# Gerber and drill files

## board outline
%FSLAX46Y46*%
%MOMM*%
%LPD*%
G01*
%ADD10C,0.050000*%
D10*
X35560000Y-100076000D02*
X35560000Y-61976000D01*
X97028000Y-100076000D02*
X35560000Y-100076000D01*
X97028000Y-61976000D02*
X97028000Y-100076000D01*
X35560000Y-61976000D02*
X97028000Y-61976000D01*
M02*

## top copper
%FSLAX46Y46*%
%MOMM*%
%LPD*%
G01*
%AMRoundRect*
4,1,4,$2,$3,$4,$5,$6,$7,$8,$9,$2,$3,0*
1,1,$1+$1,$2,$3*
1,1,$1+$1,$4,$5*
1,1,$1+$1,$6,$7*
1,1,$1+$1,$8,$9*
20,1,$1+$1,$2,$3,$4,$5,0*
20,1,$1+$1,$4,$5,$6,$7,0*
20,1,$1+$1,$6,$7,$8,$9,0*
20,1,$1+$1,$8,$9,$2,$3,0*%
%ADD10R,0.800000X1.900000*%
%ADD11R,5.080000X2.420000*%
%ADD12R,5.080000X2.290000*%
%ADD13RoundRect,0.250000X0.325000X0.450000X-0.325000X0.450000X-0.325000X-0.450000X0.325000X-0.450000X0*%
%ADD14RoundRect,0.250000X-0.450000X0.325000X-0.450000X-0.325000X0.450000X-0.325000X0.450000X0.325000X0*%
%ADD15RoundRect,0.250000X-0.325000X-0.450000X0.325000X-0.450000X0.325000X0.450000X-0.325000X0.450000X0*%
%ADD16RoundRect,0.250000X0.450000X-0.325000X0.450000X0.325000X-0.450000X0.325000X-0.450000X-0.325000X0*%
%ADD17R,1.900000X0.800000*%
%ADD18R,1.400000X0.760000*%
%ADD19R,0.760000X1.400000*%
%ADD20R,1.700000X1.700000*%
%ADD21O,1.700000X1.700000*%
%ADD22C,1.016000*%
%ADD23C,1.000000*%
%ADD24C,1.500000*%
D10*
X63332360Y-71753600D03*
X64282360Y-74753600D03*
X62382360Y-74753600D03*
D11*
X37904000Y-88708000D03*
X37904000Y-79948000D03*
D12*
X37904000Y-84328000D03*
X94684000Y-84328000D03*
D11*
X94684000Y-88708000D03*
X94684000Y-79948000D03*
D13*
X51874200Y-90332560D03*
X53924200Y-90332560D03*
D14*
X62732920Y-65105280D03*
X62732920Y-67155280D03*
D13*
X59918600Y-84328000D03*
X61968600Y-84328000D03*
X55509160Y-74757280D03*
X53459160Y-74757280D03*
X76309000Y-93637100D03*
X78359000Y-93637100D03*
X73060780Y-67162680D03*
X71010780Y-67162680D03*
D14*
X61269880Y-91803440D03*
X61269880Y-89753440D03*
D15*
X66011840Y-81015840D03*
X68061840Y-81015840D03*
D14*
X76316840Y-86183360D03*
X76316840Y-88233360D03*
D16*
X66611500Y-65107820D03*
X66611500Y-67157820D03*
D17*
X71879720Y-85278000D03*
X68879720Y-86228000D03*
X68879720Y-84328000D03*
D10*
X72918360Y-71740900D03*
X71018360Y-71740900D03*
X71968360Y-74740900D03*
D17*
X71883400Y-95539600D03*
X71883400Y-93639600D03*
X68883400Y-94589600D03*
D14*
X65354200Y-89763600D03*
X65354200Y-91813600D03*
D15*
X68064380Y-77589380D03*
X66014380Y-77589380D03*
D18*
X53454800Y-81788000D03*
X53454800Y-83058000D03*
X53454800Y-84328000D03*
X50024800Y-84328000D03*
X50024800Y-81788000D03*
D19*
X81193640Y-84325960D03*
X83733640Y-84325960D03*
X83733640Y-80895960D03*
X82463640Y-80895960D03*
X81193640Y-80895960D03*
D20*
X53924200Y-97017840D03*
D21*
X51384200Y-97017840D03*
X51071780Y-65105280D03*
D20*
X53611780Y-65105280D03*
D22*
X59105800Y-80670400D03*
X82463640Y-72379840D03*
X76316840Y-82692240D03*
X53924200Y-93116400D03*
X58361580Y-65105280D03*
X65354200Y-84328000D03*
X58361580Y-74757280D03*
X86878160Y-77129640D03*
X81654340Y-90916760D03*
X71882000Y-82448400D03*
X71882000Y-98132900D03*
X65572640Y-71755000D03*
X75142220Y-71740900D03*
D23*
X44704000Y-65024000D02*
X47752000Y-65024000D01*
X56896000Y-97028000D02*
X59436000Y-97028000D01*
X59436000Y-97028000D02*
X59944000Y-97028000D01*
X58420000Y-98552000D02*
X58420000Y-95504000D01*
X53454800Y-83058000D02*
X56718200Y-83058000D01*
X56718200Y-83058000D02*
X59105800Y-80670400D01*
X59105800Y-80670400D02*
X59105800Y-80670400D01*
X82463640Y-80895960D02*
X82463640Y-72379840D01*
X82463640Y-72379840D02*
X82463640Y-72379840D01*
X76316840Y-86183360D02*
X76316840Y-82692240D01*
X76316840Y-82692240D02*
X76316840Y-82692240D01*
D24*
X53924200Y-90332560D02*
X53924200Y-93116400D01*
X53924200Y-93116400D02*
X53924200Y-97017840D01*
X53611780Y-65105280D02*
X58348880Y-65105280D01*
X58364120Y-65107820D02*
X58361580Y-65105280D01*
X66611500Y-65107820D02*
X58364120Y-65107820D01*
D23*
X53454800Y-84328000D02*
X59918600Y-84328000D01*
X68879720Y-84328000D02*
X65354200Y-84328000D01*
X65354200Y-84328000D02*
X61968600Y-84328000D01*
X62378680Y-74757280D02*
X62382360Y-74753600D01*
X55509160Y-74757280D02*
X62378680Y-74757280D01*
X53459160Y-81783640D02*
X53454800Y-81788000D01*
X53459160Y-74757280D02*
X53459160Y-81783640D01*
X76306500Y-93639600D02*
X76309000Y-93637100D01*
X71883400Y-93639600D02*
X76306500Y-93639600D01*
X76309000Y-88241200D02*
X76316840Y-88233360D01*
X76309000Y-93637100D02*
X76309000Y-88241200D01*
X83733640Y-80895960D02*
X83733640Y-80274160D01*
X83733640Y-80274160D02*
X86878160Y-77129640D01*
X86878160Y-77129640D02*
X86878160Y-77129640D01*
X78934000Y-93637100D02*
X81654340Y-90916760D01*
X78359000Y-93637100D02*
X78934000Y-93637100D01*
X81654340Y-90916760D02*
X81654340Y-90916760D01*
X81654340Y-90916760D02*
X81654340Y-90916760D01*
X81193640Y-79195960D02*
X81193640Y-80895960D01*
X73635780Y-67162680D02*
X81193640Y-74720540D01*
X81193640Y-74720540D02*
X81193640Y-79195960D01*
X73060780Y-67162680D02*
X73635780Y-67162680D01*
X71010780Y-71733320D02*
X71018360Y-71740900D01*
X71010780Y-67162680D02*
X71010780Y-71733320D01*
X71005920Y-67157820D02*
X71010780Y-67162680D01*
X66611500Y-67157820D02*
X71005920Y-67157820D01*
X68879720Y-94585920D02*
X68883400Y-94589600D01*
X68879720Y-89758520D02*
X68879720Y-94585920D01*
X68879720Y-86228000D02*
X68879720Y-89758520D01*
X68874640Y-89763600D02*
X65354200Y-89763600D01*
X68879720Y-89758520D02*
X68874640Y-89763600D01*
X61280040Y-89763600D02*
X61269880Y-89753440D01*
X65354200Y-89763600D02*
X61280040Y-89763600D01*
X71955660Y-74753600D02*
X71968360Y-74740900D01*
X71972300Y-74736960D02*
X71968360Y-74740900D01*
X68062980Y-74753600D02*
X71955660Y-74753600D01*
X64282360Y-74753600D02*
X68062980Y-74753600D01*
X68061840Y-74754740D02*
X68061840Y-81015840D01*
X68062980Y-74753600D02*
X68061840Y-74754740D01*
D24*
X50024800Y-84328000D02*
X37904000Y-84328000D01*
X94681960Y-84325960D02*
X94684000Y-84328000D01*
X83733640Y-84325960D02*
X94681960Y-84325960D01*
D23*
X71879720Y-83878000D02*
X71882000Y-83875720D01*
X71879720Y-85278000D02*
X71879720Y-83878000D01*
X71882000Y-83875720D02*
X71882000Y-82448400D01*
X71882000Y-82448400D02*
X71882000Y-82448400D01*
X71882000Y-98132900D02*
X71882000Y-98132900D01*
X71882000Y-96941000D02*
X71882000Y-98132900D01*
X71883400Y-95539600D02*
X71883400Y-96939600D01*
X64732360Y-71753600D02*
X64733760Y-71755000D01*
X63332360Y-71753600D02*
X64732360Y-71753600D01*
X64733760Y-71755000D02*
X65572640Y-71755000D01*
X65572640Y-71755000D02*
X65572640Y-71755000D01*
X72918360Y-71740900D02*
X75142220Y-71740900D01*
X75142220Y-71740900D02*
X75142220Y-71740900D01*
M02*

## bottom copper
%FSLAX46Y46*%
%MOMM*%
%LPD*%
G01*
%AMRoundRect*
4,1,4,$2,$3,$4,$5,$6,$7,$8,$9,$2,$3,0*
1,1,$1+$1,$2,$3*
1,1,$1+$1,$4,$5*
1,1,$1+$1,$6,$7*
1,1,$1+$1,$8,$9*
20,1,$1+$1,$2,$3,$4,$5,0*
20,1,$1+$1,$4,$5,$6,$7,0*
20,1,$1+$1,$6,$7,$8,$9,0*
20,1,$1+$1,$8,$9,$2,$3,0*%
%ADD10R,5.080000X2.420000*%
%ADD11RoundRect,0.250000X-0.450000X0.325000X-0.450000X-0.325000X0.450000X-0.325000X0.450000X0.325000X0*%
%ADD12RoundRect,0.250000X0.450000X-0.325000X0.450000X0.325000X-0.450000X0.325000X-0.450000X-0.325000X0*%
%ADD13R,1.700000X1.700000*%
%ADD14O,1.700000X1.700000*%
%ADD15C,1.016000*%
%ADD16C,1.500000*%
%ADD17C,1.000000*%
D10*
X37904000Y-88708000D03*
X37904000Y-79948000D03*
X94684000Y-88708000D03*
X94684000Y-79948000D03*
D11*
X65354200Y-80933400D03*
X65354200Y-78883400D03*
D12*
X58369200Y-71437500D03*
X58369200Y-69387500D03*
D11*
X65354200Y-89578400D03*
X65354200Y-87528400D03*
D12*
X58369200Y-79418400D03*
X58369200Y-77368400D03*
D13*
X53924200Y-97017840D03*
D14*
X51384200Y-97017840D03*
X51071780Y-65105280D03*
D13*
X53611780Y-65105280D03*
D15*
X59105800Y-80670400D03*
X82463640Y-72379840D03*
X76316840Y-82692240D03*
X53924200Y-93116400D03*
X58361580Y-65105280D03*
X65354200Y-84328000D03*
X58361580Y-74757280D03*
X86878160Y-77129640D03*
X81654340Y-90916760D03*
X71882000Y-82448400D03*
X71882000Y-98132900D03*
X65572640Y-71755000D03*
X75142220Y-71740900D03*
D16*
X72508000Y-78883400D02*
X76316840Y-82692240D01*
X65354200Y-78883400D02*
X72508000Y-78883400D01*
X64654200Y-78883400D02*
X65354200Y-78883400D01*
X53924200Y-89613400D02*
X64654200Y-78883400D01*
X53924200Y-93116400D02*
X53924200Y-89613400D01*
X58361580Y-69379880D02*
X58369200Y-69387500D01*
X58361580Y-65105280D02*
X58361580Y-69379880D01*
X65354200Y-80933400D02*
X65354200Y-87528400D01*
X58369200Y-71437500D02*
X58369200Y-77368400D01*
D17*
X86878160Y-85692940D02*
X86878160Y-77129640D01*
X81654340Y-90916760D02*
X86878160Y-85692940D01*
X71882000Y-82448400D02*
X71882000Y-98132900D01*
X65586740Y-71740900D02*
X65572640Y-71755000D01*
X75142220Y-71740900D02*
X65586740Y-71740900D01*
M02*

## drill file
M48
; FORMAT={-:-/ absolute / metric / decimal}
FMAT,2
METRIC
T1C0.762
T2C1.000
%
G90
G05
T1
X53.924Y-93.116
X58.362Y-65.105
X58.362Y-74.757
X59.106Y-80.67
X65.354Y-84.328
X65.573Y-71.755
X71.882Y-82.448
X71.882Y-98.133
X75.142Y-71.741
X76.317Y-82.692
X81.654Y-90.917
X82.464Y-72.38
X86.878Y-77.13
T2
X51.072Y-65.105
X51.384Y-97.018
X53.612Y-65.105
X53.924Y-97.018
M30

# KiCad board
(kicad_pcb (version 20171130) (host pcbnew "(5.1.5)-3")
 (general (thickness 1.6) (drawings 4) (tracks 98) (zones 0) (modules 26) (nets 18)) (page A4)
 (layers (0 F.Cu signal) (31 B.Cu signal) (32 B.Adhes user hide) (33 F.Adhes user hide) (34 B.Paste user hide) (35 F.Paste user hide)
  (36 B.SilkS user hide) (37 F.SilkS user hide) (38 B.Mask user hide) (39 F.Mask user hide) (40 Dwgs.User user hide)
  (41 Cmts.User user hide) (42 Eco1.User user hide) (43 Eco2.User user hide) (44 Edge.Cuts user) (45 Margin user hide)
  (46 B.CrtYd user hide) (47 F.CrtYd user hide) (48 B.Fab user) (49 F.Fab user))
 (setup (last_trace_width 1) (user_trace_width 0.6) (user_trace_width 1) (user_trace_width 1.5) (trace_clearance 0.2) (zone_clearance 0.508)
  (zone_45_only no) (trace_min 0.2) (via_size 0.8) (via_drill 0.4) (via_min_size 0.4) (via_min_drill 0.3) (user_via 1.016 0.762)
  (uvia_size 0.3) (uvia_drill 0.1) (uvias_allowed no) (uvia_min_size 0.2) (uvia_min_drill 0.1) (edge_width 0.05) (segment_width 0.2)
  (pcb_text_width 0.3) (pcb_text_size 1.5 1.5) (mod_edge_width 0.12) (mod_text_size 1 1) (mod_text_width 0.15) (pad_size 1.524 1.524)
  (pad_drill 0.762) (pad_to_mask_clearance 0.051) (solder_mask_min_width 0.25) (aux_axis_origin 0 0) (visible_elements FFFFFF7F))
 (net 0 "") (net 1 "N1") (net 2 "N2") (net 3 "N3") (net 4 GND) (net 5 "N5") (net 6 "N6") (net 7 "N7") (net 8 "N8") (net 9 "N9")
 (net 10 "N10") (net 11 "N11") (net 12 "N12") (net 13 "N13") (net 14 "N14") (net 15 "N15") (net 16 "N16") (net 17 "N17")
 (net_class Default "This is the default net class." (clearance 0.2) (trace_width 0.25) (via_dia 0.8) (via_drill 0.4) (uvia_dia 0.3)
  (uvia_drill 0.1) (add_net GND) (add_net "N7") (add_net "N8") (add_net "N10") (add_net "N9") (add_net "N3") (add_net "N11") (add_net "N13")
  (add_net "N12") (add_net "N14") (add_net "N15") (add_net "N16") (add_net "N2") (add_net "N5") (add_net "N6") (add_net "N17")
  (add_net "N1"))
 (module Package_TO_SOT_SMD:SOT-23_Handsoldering (layer F.Cu) (at 63.33236 73.2536 90)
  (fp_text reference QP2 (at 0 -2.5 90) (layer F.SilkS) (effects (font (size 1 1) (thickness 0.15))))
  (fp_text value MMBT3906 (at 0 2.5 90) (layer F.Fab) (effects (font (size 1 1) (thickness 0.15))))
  (pad 3 smd rect (at 1.5 0 90) (size 1.9 0.8) (layers F.Cu F.Paste F.Mask) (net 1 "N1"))
  (pad 2 smd rect (at -1.5 0.95 90) (size 1.9 0.8) (layers F.Cu F.Paste F.Mask) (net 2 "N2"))
  (pad 1 smd rect (at -1.5 -0.95 90) (size 1.9 0.8) (layers F.Cu F.Paste F.Mask) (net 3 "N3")))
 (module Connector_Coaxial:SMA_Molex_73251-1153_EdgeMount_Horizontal (layer F.Cu) (at 39.624 84.328)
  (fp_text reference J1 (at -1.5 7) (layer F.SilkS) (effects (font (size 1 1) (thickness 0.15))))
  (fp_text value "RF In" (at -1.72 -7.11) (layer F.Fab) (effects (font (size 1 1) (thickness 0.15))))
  (pad 2 smd rect (at -1.72 4.38) (size 5.08 2.42) (layers B.Cu B.Paste B.Mask) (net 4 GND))
  (pad 2 smd rect (at -1.72 -4.38) (size 5.08 2.42) (layers B.Cu B.Paste B.Mask) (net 4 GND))
  (pad 2 smd rect (at -1.72 4.38) (size 5.08 2.42) (layers F.Cu F.Paste F.Mask) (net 4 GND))
  (pad 2 smd rect (at -1.72 -4.38) (size 5.08 2.42) (layers F.Cu F.Paste F.Mask) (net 4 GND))
  (pad 1 smd rect (at -1.72 0) (size 5.08 2.29) (layers F.Cu F.Paste F.Mask) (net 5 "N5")))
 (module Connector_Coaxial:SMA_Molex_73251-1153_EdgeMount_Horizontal (layer F.Cu) (at 92.964 84.328 180)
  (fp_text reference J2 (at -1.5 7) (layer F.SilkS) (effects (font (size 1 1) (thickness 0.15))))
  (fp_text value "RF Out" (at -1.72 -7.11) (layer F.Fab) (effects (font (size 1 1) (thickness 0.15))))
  (pad 1 smd rect (at -1.72 0 180) (size 5.08 2.29) (layers F.Cu F.Paste F.Mask) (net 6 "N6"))
  (pad 2 smd rect (at -1.72 -4.38 180) (size 5.08 2.42) (layers F.Cu F.Paste F.Mask) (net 4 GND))
  (pad 2 smd rect (at -1.72 4.38 180) (size 5.08 2.42) (layers F.Cu F.Paste F.Mask) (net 4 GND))
  (pad 2 smd rect (at -1.72 -4.38 180) (size 5.08 2.42) (layers B.Cu B.Paste B.Mask) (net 4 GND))
  (pad 2 smd rect (at -1.72 4.38 180) (size 5.08 2.42) (layers B.Cu B.Paste B.Mask) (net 4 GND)))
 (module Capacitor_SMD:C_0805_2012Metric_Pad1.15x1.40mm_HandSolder (layer F.Cu) (at 52.8992 90.33256 180)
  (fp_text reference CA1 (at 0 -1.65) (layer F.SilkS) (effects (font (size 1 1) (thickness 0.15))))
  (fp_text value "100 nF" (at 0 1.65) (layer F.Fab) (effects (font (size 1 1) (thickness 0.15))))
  (pad 2 smd roundrect (at 1.025 0 180) (size 1.15 1.4) (layers F.Cu F.Paste F.Mask) (roundrect_rratio 0.217391) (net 4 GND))
  (pad 1 smd roundrect (at -1.025 0 180) (size 1.15 1.4) (layers F.Cu F.Paste F.Mask) (roundrect_rratio 0.217391) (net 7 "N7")))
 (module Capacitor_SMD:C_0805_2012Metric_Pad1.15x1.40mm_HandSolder (layer F.Cu) (at 62.73292 66.13028 270)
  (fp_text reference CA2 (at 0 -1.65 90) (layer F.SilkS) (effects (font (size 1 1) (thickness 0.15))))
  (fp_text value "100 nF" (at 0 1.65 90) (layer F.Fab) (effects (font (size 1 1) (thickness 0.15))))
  (pad 1 smd roundrect (at -1.025 0 270) (size 1.15 1.4) (layers F.Cu F.Paste F.Mask) (roundrect_rratio 0.217391) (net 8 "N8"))
  (pad 2 smd roundrect (at 1.025 0 270) (size 1.15 1.4) (layers F.Cu F.Paste F.Mask) (roundrect_rratio 0.217391) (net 4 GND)))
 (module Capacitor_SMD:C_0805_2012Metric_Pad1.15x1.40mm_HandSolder (layer F.Cu) (at 60.9436 84.328 180)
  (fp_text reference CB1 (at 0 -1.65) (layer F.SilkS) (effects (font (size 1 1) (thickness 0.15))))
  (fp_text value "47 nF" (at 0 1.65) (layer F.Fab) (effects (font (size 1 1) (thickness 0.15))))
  (pad 2 smd roundrect (at 1.025 0 180) (size 1.15 1.4) (layers F.Cu F.Paste F.Mask) (roundrect_rratio 0.217391) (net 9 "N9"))
  (pad 1 smd roundrect (at -1.025 0 180) (size 1.15 1.4) (layers F.Cu F.Paste F.Mask) (roundrect_rratio 0.217391) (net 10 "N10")))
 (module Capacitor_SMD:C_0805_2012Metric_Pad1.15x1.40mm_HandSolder (layer F.Cu) (at 54.48416 74.75728 180)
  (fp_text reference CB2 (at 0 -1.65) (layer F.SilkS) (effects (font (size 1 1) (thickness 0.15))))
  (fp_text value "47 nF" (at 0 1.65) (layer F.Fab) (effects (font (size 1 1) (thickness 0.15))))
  (pad 1 smd roundrect (at -1.025 0 180) (size 1.15 1.4) (layers F.Cu F.Paste F.Mask) (roundrect_rratio 0.217391) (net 3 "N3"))
  (pad 2 smd roundrect (at 1.025 0 180) (size 1.15 1.4) (layers F.Cu F.Paste F.Mask) (roundrect_rratio 0.217391) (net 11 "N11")))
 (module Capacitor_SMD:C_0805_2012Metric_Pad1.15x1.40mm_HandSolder (layer F.Cu) (at 77.334 93.6371 180)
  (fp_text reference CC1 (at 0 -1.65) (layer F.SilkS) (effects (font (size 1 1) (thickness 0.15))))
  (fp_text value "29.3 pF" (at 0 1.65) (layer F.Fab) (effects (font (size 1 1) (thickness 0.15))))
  (pad 2 smd roundrect (at 1.025 0 180) (size 1.15 1.4) (layers F.Cu F.Paste F.Mask) (roundrect_rratio 0.217391) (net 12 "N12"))
  (pad 1 smd roundrect (at -1.025 0 180) (size 1.15 1.4) (layers F.Cu F.Paste F.Mask) (roundrect_rratio 0.217391) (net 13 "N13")))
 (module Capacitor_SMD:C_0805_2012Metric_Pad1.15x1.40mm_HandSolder (layer F.Cu) (at 72.03578 67.16268 180)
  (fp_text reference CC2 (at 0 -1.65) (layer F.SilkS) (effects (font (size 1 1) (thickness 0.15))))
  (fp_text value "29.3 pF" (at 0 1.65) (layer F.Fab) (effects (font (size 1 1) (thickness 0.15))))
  (pad 1 smd roundrect (at -1.025 0 180) (size 1.15 1.4) (layers F.Cu F.Paste F.Mask) (roundrect_rratio 0.217391) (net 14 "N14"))
  (pad 2 smd roundrect (at 1.025 0 180) (size 1.15 1.4) (layers F.Cu F.Paste F.Mask) (roundrect_rratio 0.217391) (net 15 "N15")))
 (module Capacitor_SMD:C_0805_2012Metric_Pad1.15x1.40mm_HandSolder (layer F.Cu) (at 61.26988 90.77844 270)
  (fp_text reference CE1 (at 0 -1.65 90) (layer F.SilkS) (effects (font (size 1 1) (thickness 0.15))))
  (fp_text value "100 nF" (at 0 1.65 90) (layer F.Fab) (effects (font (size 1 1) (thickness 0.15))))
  (pad 2 smd roundrect (at 1.025 0 270) (size 1.15 1.4) (layers F.Cu F.Paste F.Mask) (roundrect_rratio 0.217391) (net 4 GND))
  (pad 1 smd roundrect (at -1.025 0 270) (size 1.15 1.4) (layers F.Cu F.Paste F.Mask) (roundrect_rratio 0.217391) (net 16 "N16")))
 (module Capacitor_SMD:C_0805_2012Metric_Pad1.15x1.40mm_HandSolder (layer F.Cu) (at 67.03684 81.01584)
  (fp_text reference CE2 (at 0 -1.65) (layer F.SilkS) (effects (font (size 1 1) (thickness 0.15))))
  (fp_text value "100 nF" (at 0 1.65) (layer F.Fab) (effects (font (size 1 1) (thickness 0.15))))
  (pad 1 smd roundrect (at -1.025 0) (size 1.15 1.4) (layers F.Cu F.Paste F.Mask) (roundrect_rratio 0.217391) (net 4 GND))
  (pad 2 smd roundrect (at 1.025 0) (size 1.15 1.4) (layers F.Cu F.Paste F.Mask) (roundrect_rratio 0.217391) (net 2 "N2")))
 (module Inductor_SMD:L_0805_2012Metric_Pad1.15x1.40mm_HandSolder (layer F.Cu) (at 76.31684 87.20836 270)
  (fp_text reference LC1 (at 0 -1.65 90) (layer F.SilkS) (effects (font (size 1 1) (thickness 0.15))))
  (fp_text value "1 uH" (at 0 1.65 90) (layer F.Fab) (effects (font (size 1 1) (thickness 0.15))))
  (pad 1 smd roundrect (at -1.025 0 270) (size 1.15 1.4) (layers F.Cu F.Paste F.Mask) (roundrect_rratio 0.217391) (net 7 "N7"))
  (pad 2 smd roundrect (at 1.025 0 270) (size 1.15 1.4) (layers F.Cu F.Paste F.Mask) (roundrect_rratio 0.217391) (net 12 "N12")))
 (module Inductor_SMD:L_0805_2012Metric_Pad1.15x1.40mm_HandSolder (layer F.Cu) (at 66.6115 66.13282 90)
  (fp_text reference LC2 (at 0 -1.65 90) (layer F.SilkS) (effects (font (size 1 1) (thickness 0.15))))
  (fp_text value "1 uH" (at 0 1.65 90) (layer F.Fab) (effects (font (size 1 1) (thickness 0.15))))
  (pad 2 smd roundrect (at 1.025 0 90) (size 1.15 1.4) (layers F.Cu F.Paste F.Mask) (roundrect_rratio 0.217391) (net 8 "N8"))
  (pad 1 smd roundrect (at -1.025 0 90) (size 1.15 1.4) (layers F.Cu F.Paste F.Mask) (roundrect_rratio 0.217391) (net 15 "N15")))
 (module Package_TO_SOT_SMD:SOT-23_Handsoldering (layer F.Cu) (at 70.37972 85.278)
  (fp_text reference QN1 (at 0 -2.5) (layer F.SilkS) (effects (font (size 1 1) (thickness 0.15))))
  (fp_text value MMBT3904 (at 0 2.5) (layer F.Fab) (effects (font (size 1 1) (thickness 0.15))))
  (pad 3 smd rect (at 1.5 0) (size 1.9 0.8) (layers F.Cu F.Paste F.Mask) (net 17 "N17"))
  (pad 2 smd rect (at -1.5 0.95) (size 1.9 0.8) (layers F.Cu F.Paste F.Mask) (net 16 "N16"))
  (pad 1 smd rect (at -1.5 -0.95) (size 1.9 0.8) (layers F.Cu F.Paste F.Mask) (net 10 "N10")))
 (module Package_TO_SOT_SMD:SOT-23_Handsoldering (layer F.Cu) (at 71.96836 73.2409 270)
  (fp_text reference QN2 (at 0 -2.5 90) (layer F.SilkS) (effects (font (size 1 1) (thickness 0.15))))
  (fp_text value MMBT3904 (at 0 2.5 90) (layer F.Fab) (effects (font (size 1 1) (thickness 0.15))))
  (pad 1 smd rect (at -1.5 -0.95 270) (size 1.9 0.8) (layers F.Cu F.Paste F.Mask) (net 1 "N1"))
  (pad 2 smd rect (at -1.5 0.95 270) (size 1.9 0.8) (layers F.Cu F.Paste F.Mask) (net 15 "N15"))
  (pad 3 smd rect (at 1.5 0 270) (size 1.9 0.8) (layers F.Cu F.Paste F.Mask) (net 2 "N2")))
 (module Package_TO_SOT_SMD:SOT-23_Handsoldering (layer F.Cu) (at 70.3834 94.5896 180)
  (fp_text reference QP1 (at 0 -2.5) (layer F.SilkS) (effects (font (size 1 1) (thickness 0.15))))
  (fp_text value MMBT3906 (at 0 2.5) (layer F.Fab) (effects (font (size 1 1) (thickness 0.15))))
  (pad 1 smd rect (at -1.5 -0.95 180) (size 1.9 0.8) (layers F.Cu F.Paste F.Mask) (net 17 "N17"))
  (pad 2 smd rect (at -1.5 0.95 180) (size 1.9 0.8) (layers F.Cu F.Paste F.Mask) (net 12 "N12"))
  (pad 3 smd rect (at 1.5 0 180) (size 1.9 0.8) (layers F.Cu F.Paste F.Mask) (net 16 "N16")))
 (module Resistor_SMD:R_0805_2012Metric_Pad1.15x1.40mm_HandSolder (layer B.Cu) (at 65.3542 79.9084 270)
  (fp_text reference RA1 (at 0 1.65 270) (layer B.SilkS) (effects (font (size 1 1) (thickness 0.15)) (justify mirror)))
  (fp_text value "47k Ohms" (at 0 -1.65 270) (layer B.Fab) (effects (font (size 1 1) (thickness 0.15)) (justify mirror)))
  (pad 2 smd roundrect (at 1.025 0 270) (size 1.15 1.4) (layers B.Cu B.Paste B.Mask) (roundrect_rratio 0.217391) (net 10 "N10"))
  (pad 1 smd roundrect (at -1.025 0 270) (size 1.15 1.4) (layers B.Cu B.Paste B.Mask) (roundrect_rratio 0.217391) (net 7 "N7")))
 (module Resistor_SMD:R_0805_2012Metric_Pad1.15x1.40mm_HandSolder (layer B.Cu) (at 58.3692 70.4125 90)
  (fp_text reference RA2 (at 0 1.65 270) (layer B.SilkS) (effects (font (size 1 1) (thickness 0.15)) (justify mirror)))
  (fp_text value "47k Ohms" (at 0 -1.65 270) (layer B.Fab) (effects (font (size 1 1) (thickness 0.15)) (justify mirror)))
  (pad 1 smd roundrect (at -1.025 0 90) (size 1.15 1.4) (layers B.Cu B.Paste B.Mask) (roundrect_rratio 0.217391) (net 3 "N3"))
  (pad 2 smd roundrect (at 1.025 0 90) (size 1.15 1.4) (layers B.Cu B.Paste B.Mask) (roundrect_rratio 0.217391) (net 8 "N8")))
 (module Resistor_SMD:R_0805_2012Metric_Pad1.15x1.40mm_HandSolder (layer B.Cu) (at 65.3542 88.5534 270)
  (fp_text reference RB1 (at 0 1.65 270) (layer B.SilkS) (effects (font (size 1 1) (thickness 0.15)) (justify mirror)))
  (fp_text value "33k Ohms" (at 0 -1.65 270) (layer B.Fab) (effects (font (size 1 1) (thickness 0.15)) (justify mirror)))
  (pad 2 smd roundrect (at 1.025 0 270) (size 1.15 1.4) (layers B.Cu B.Paste B.Mask) (roundrect_rratio 0.217391) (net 4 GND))
  (pad 1 smd roundrect (at -1.025 0 270) (size 1.15 1.4) (layers B.Cu B.Paste B.Mask) (roundrect_rratio 0.217391) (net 10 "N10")))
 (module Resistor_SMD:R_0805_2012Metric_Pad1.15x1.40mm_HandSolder (layer B.Cu) (at 58.3692 78.3934 90)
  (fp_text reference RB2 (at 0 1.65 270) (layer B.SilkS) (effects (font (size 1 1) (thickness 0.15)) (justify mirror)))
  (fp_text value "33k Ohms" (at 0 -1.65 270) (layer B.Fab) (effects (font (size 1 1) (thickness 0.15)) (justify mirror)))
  (pad 1 smd roundrect (at -1.025 0 90) (size 1.15 1.4) (layers B.Cu B.Paste B.Mask) (roundrect_rratio 0.217391) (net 4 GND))
  (pad 2 smd roundrect (at 1.025 0 90) (size 1.15 1.4) (layers B.Cu B.Paste B.Mask) (roundrect_rratio 0.217391) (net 3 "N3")))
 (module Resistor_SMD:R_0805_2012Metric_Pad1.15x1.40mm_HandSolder (layer F.Cu) (at 65.3542 90.7886 270)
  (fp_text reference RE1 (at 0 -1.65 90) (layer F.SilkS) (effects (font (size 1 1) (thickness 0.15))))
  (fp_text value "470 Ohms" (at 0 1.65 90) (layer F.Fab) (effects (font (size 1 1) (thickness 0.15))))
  (pad 1 smd roundrect (at -1.025 0 270) (size 1.15 1.4) (layers F.Cu F.Paste F.Mask) (roundrect_rratio 0.217391) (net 16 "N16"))
  (pad 2 smd roundrect (at 1.025 0 270) (size 1.15 1.4) (layers F.Cu F.Paste F.Mask) (roundrect_rratio 0.217391) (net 4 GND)))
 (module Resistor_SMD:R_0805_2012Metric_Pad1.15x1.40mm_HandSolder (layer F.Cu) (at 67.03938 77.58938)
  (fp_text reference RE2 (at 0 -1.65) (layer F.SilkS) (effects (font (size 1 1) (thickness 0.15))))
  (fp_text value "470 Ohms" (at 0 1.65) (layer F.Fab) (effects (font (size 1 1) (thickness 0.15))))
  (pad 2 smd roundrect (at 1.025 0) (size 1.15 1.4) (layers F.Cu F.Paste F.Mask) (roundrect_rratio 0.217391) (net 2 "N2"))
  (pad 1 smd roundrect (at -1.025 0) (size 1.15 1.4) (layers F.Cu F.Paste F.Mask) (roundrect_rratio 0.217391) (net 4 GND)))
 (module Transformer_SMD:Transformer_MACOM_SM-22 (layer F.Cu) (at 51.7398 83.058)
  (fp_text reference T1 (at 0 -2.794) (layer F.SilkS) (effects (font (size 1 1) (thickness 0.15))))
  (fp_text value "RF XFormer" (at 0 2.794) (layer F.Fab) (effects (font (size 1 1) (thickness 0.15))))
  (pad 5 smd rect (at 1.715 -1.27) (size 1.4 0.76) (layers F.Cu F.Paste F.Mask) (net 11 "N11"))
  (pad 4 smd rect (at 1.715 0) (size 1.4 0.76) (layers F.Cu F.Paste F.Mask) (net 4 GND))
  (pad 3 smd rect (at 1.715 1.27) (size 1.4 0.76) (layers F.Cu F.Paste F.Mask) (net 9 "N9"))
  (pad 2 smd rect (at -1.715 1.27) (size 1.4 0.76) (layers F.Cu F.Paste F.Mask) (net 5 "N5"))
  (pad 1 smd rect (at -1.715 -1.27) (size 1.4 0.76) (layers F.Cu F.Paste F.Mask) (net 4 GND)))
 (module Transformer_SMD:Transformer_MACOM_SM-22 (layer F.Cu) (at 82.46364 82.61096 90)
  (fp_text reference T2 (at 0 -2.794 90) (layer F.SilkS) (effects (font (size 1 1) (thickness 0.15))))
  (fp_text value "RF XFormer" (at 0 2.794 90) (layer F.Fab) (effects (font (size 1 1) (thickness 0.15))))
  (pad 1 smd rect (at -1.715 -1.27 90) (size 1.4 0.76) (layers F.Cu F.Paste F.Mask) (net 4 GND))
  (pad 2 smd rect (at -1.715 1.27 90) (size 1.4 0.76) (layers F.Cu F.Paste F.Mask) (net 6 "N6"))
  (pad 3 smd rect (at 1.715 1.27 90) (size 1.4 0.76) (layers F.Cu F.Paste F.Mask) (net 13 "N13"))
  (pad 4 smd rect (at 1.715 0 90) (size 1.4 0.76) (layers F.Cu F.Paste F.Mask) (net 4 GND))
  (pad 5 smd rect (at 1.715 -1.27 90) (size 1.4 0.76) (layers F.Cu F.Paste F.Mask) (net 14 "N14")))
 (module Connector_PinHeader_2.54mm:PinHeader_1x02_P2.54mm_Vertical (layer F.Cu) (at 53.9242 97.01784 270)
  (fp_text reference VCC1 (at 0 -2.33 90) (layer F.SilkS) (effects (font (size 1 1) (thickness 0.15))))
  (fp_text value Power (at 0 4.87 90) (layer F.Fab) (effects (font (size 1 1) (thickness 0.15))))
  (pad 1 thru_hole rect (at 0 0 270) (size 1.7 1.7) (drill 1) (layers *.Cu *.Mask) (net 7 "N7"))
  (pad 2 thru_hole oval (at 0 2.54 270) (size 1.7 1.7) (drill 1) (layers *.Cu *.Mask) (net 4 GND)))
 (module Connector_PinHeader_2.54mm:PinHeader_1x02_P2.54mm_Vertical (layer F.Cu) (at 53.61178 65.10528 270)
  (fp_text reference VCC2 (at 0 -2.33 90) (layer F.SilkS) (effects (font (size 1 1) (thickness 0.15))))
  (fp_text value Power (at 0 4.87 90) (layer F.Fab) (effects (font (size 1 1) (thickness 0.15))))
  (pad 2 thru_hole oval (at 0 2.54 270) (size 1.7 1.7) (drill 1) (layers *.Cu *.Mask) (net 4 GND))
  (pad 1 thru_hole rect (at 0 0 270) (size 1.7 1.7) (drill 1) (layers *.Cu *.Mask) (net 8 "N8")))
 (gr_line (start 35.56 100.076) (end 35.56 61.976) (layer Edge.Cuts) (width 0.05))
 (gr_line (start 97.028 100.076) (end 35.56 100.076) (layer Edge.Cuts) (width 0.05))
 (gr_line (start 97.028 61.976) (end 97.028 100.076) (layer Edge.Cuts) (width 0.05))
 (gr_line (start 35.56 61.976) (end 97.028 61.976) (layer Edge.Cuts) (width 0.05))
 (segment (start 44.704 65.024) (end 47.752 65.024) (width 1) (layer F.Cu) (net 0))
 (segment (start 56.896 97.028) (end 59.436 97.028) (width 1) (layer F.Cu) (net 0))
 (segment (start 59.436 97.028) (end 59.944 97.028) (width 1) (layer F.Cu) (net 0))
 (segment (start 58.42 98.552) (end 58.42 95.504) (width 1) (layer F.Cu) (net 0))
 (segment (start 53.4548 83.058) (end 56.7182 83.058) (width 1) (layer F.Cu) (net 4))
 (segment (start 56.7182 83.058) (end 59.1058 80.6704) (width 1) (layer F.Cu) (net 4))
 (segment (start 59.1058 80.6704) (end 59.1058 80.6704) (width 1) (layer F.Cu) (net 4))
 (via (at 59.1058 80.6704) (size 1.016) (drill 0.762) (layers F.Cu B.Cu) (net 4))
 (segment (start 82.46364 80.89596) (end 82.46364 72.37984) (width 1) (layer F.Cu) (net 4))
 (segment (start 82.46364 72.37984) (end 82.46364 72.37984) (width 1) (layer F.Cu) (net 4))
 (via (at 82.46364 72.37984) (size 1.016) (drill 0.762) (layers F.Cu B.Cu) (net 4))
 (segment (start 76.31684 86.18336) (end 76.31684 82.69224) (width 1) (layer F.Cu) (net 7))
 (segment (start 76.31684 82.69224) (end 76.31684 82.69224) (width 1) (layer F.Cu) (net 7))
 (via (at 76.31684 82.69224) (size 1.016) (drill 0.762) (layers F.Cu B.Cu) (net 7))
 (segment (start 72.508 78.8834) (end 76.31684 82.69224) (width 1.5) (layer B.Cu) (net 7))
 (segment (start 65.3542 78.8834) (end 72.508 78.8834) (width 1.5) (layer B.Cu) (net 7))
 (segment (start 53.9242 90.33256) (end 53.9242 93.1164) (width 1.5) (layer F.Cu) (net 7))
 (segment (start 53.9242 93.1164) (end 53.9242 97.01784) (width 1.5) (layer F.Cu) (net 7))
 (via (at 53.9242 93.1164) (size 1.016) (drill 0.762) (layers F.Cu B.Cu) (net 7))
 (segment (start 64.6542 78.8834) (end 65.3542 78.8834) (width 1.5) (layer B.Cu) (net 7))
 (segment (start 53.9242 89.6134) (end 64.6542 78.8834) (width 1.5) (layer B.Cu) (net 7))
 (segment (start 53.9242 93.1164) (end 53.9242 89.6134) (width 1.5) (layer B.Cu) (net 7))
 (segment (start 53.61178 65.10528) (end 58.34888 65.10528) (width 1.5) (layer F.Cu) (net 8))
 (via (at 58.36158 65.10528) (size 1.016) (drill 0.762) (layers F.Cu B.Cu) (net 8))
 (segment (start 58.36158 69.37988) (end 58.3692 69.3875) (width 1.5) (layer B.Cu) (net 8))
 (segment (start 58.36158 65.10528) (end 58.36158 69.37988) (width 1.5) (layer B.Cu) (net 8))
 (segment (start 58.36412 65.10782) (end 58.36158 65.10528) (width 1.5) (layer F.Cu) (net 8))
 (segment (start 66.6115 65.10782) (end 58.36412 65.10782) (width 1.5) (layer F.Cu) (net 8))
 (segment (start 53.4548 84.328) (end 59.9186 84.328) (width 1) (layer F.Cu) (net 9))
 (segment (start 68.87972 84.328) (end 65.3542 84.328) (width 1) (layer F.Cu) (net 10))
 (segment (start 65.3542 84.328) (end 61.9686 84.328) (width 1) (layer F.Cu) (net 10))
 (via (at 65.3542 84.328) (size 1.016) (drill 0.762) (layers F.Cu B.Cu) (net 10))
 (segment (start 65.3542 80.9334) (end 65.3542 87.5284) (width 1.5) (layer B.Cu) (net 10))
 (via (at 58.36158 74.75728) (size 1.016) (drill 0.762) (layers F.Cu B.Cu) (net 3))
 (segment (start 58.3692 71.4375) (end 58.3692 77.3684) (width 1.5) (layer B.Cu) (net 3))
 (segment (start 62.37868 74.75728) (end 62.38236 74.7536) (width 1) (layer F.Cu) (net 3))
 (segment (start 55.50916 74.75728) (end 62.37868 74.75728) (width 1) (layer F.Cu) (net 3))
 (segment (start 53.45916 81.78364) (end 53.4548 81.788) (width 1) (layer F.Cu) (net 11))
 (segment (start 53.45916 74.75728) (end 53.45916 81.78364) (width 1) (layer F.Cu) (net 11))
 (segment (start 76.3065 93.6396) (end 76.309 93.6371) (width 1) (layer F.Cu) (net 12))
 (segment (start 71.8834 93.6396) (end 76.3065 93.6396) (width 1) (layer F.Cu) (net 12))
 (segment (start 76.309 88.2412) (end 76.31684 88.23336) (width 1) (layer F.Cu) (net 12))
 (segment (start 76.309 93.6371) (end 76.309 88.2412) (width 1) (layer F.Cu) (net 12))
 (segment (start 83.73364 80.89596) (end 83.73364 80.27416) (width 1) (layer F.Cu) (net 13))
 (segment (start 83.73364 80.27416) (end 86.87816 77.12964) (width 1) (layer F.Cu) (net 13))
 (segment (start 86.87816 77.12964) (end 86.87816 77.12964) (width 1) (layer F.Cu) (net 13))
 (via (at 86.87816 77.12964) (size 1.016) (drill 0.762) (layers F.Cu B.Cu) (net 13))
 (segment (start 78.934 93.6371) (end 81.65434 90.91676) (width 1) (layer F.Cu) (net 13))
 (segment (start 78.359 93.6371) (end 78.934 93.6371) (width 1) (layer F.Cu) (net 13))
 (segment (start 81.65434 90.91676) (end 81.65434 90.91676) (width 1) (layer F.Cu) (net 13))
 (segment (start 81.65434 90.91676) (end 81.65434 90.91676) (width 1) (layer F.Cu) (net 13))
 (via (at 81.65434 90.91676) (size 1.016) (drill 0.762) (layers F.Cu B.Cu) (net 13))
 (segment (start 86.87816 85.69294) (end 86.87816 77.12964) (width 1) (layer B.Cu) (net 13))
 (segment (start 81.65434 90.91676) (end 86.87816 85.69294) (width 1) (layer B.Cu) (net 13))
 (segment (start 81.19364 79.19596) (end 81.19364 80.89596) (width 1) (layer F.Cu) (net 14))
 (segment (start 73.63578 67.16268) (end 81.19364 74.72054) (width 1) (layer F.Cu) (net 14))
 (segment (start 81.19364 74.72054) (end 81.19364 79.19596) (width 1) (layer F.Cu) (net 14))
 (segment (start 73.06078 67.16268) (end 73.63578 67.16268) (width 1) (layer F.Cu) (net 14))
 (segment (start 71.01078 71.73332) (end 71.01836 71.7409) (width 1) (layer F.Cu) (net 15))
 (segment (start 71.01078 67.16268) (end 71.01078 71.73332) (width 1) (layer F.Cu) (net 15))
 (segment (start 71.00592 67.15782) (end 71.01078 67.16268) (width 1) (layer F.Cu) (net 15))
 (segment (start 66.6115 67.15782) (end 71.00592 67.15782) (width 1) (layer F.Cu) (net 15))
 (segment (start 68.87972 94.58592) (end 68.8834 94.5896) (width 1) (layer F.Cu) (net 16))
 (segment (start 68.87972 89.75852) (end 68.87972 94.58592) (width 1) (layer F.Cu) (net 16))
 (segment (start 68.87972 86.228) (end 68.87972 89.75852) (width 1) (layer F.Cu) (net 16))
 (segment (start 68.87464 89.7636) (end 65.3542 89.7636) (width 1) (layer F.Cu) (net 16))
 (segment (start 68.87972 89.75852) (end 68.87464 89.7636) (width 1) (layer F.Cu) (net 16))
 (segment (start 61.28004 89.7636) (end 61.26988 89.75344) (width 1) (layer F.Cu) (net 16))
 (segment (start 65.3542 89.7636) (end 61.28004 89.7636) (width 1) (layer F.Cu) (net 16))
 (segment (start 71.95566 74.7536) (end 71.96836 74.7409) (width 1) (layer F.Cu) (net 2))
 (segment (start 71.9723 74.73696) (end 71.96836 74.7409) (width 1) (layer F.Cu) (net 2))
 (segment (start 68.06298 74.7536) (end 71.95566 74.7536) (width 1) (layer F.Cu) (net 2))
 (segment (start 64.28236 74.7536) (end 68.06298 74.7536) (width 1) (layer F.Cu) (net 2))
 (segment (start 68.06184 74.75474) (end 68.06184 81.01584) (width 1) (layer F.Cu) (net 2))
 (segment (start 68.06298 74.7536) (end 68.06184 74.75474) (width 1) (layer F.Cu) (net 2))
 (segment (start 50.0248 84.328) (end 37.904 84.328) (width 1.5) (layer F.Cu) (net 5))
 (segment (start 94.68196 84.32596) (end 94.684 84.328) (width 1.5) (layer F.Cu) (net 6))
 (segment (start 83.73364 84.32596) (end 94.68196 84.32596) (width 1.5) (layer F.Cu) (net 6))
 (segment (start 71.87972 83.878) (end 71.882 83.87572) (width 1) (layer F.Cu) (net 17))
 (segment (start 71.87972 85.278) (end 71.87972 83.878) (width 1) (layer F.Cu) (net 17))
 (segment (start 71.882 83.87572) (end 71.882 82.4484) (width 1) (layer F.Cu) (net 17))
 (segment (start 71.882 82.4484) (end 71.882 82.4484) (width 1) (layer F.Cu) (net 17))
 (via (at 71.882 82.4484) (size 1.016) (drill 0.762) (layers F.Cu B.Cu) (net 17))
 (segment (start 71.882 98.1329) (end 71.882 98.1329) (width 1) (layer F.Cu) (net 17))
 (via (at 71.882 98.1329) (size 1.016) (drill 0.762) (layers F.Cu B.Cu) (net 17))
 (segment (start 71.882 82.4484) (end 71.882 98.1329) (width 1) (layer B.Cu) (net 17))
 (segment (start 71.882 96.941) (end 71.882 98.1329) (width 1) (layer F.Cu) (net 17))
 (segment (start 71.8834 95.5396) (end 71.8834 96.9396) (width 1) (layer F.Cu) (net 17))
 (segment (start 64.73236 71.7536) (end 64.73376 71.755) (width 1) (layer F.Cu) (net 1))
 (segment (start 63.33236 71.7536) (end 64.73236 71.7536) (width 1) (layer F.Cu) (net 1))
 (segment (start 64.73376 71.755) (end 65.57264 71.755) (width 1) (layer F.Cu) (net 1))
 (segment (start 65.57264 71.755) (end 65.57264 71.755) (width 1) (layer F.Cu) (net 1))
 (via (at 65.57264 71.755) (size 1.016) (drill 0.762) (layers F.Cu B.Cu) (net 1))
 (segment (start 72.91836 71.7409) (end 75.14222 71.7409) (width 1) (layer F.Cu) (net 1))
 (segment (start 75.14222 71.7409) (end 75.14222 71.7409) (width 1) (layer F.Cu) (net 1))
 (via (at 75.14222 71.7409) (size 1.016) (drill 0.762) (layers F.Cu B.Cu) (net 1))
 (segment (start 65.58674 71.7409) (end 65.57264 71.755) (width 1) (layer B.Cu) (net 1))
 (segment (start 75.14222 71.7409) (end 65.58674 71.7409) (width 1) (layer B.Cu) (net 1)))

